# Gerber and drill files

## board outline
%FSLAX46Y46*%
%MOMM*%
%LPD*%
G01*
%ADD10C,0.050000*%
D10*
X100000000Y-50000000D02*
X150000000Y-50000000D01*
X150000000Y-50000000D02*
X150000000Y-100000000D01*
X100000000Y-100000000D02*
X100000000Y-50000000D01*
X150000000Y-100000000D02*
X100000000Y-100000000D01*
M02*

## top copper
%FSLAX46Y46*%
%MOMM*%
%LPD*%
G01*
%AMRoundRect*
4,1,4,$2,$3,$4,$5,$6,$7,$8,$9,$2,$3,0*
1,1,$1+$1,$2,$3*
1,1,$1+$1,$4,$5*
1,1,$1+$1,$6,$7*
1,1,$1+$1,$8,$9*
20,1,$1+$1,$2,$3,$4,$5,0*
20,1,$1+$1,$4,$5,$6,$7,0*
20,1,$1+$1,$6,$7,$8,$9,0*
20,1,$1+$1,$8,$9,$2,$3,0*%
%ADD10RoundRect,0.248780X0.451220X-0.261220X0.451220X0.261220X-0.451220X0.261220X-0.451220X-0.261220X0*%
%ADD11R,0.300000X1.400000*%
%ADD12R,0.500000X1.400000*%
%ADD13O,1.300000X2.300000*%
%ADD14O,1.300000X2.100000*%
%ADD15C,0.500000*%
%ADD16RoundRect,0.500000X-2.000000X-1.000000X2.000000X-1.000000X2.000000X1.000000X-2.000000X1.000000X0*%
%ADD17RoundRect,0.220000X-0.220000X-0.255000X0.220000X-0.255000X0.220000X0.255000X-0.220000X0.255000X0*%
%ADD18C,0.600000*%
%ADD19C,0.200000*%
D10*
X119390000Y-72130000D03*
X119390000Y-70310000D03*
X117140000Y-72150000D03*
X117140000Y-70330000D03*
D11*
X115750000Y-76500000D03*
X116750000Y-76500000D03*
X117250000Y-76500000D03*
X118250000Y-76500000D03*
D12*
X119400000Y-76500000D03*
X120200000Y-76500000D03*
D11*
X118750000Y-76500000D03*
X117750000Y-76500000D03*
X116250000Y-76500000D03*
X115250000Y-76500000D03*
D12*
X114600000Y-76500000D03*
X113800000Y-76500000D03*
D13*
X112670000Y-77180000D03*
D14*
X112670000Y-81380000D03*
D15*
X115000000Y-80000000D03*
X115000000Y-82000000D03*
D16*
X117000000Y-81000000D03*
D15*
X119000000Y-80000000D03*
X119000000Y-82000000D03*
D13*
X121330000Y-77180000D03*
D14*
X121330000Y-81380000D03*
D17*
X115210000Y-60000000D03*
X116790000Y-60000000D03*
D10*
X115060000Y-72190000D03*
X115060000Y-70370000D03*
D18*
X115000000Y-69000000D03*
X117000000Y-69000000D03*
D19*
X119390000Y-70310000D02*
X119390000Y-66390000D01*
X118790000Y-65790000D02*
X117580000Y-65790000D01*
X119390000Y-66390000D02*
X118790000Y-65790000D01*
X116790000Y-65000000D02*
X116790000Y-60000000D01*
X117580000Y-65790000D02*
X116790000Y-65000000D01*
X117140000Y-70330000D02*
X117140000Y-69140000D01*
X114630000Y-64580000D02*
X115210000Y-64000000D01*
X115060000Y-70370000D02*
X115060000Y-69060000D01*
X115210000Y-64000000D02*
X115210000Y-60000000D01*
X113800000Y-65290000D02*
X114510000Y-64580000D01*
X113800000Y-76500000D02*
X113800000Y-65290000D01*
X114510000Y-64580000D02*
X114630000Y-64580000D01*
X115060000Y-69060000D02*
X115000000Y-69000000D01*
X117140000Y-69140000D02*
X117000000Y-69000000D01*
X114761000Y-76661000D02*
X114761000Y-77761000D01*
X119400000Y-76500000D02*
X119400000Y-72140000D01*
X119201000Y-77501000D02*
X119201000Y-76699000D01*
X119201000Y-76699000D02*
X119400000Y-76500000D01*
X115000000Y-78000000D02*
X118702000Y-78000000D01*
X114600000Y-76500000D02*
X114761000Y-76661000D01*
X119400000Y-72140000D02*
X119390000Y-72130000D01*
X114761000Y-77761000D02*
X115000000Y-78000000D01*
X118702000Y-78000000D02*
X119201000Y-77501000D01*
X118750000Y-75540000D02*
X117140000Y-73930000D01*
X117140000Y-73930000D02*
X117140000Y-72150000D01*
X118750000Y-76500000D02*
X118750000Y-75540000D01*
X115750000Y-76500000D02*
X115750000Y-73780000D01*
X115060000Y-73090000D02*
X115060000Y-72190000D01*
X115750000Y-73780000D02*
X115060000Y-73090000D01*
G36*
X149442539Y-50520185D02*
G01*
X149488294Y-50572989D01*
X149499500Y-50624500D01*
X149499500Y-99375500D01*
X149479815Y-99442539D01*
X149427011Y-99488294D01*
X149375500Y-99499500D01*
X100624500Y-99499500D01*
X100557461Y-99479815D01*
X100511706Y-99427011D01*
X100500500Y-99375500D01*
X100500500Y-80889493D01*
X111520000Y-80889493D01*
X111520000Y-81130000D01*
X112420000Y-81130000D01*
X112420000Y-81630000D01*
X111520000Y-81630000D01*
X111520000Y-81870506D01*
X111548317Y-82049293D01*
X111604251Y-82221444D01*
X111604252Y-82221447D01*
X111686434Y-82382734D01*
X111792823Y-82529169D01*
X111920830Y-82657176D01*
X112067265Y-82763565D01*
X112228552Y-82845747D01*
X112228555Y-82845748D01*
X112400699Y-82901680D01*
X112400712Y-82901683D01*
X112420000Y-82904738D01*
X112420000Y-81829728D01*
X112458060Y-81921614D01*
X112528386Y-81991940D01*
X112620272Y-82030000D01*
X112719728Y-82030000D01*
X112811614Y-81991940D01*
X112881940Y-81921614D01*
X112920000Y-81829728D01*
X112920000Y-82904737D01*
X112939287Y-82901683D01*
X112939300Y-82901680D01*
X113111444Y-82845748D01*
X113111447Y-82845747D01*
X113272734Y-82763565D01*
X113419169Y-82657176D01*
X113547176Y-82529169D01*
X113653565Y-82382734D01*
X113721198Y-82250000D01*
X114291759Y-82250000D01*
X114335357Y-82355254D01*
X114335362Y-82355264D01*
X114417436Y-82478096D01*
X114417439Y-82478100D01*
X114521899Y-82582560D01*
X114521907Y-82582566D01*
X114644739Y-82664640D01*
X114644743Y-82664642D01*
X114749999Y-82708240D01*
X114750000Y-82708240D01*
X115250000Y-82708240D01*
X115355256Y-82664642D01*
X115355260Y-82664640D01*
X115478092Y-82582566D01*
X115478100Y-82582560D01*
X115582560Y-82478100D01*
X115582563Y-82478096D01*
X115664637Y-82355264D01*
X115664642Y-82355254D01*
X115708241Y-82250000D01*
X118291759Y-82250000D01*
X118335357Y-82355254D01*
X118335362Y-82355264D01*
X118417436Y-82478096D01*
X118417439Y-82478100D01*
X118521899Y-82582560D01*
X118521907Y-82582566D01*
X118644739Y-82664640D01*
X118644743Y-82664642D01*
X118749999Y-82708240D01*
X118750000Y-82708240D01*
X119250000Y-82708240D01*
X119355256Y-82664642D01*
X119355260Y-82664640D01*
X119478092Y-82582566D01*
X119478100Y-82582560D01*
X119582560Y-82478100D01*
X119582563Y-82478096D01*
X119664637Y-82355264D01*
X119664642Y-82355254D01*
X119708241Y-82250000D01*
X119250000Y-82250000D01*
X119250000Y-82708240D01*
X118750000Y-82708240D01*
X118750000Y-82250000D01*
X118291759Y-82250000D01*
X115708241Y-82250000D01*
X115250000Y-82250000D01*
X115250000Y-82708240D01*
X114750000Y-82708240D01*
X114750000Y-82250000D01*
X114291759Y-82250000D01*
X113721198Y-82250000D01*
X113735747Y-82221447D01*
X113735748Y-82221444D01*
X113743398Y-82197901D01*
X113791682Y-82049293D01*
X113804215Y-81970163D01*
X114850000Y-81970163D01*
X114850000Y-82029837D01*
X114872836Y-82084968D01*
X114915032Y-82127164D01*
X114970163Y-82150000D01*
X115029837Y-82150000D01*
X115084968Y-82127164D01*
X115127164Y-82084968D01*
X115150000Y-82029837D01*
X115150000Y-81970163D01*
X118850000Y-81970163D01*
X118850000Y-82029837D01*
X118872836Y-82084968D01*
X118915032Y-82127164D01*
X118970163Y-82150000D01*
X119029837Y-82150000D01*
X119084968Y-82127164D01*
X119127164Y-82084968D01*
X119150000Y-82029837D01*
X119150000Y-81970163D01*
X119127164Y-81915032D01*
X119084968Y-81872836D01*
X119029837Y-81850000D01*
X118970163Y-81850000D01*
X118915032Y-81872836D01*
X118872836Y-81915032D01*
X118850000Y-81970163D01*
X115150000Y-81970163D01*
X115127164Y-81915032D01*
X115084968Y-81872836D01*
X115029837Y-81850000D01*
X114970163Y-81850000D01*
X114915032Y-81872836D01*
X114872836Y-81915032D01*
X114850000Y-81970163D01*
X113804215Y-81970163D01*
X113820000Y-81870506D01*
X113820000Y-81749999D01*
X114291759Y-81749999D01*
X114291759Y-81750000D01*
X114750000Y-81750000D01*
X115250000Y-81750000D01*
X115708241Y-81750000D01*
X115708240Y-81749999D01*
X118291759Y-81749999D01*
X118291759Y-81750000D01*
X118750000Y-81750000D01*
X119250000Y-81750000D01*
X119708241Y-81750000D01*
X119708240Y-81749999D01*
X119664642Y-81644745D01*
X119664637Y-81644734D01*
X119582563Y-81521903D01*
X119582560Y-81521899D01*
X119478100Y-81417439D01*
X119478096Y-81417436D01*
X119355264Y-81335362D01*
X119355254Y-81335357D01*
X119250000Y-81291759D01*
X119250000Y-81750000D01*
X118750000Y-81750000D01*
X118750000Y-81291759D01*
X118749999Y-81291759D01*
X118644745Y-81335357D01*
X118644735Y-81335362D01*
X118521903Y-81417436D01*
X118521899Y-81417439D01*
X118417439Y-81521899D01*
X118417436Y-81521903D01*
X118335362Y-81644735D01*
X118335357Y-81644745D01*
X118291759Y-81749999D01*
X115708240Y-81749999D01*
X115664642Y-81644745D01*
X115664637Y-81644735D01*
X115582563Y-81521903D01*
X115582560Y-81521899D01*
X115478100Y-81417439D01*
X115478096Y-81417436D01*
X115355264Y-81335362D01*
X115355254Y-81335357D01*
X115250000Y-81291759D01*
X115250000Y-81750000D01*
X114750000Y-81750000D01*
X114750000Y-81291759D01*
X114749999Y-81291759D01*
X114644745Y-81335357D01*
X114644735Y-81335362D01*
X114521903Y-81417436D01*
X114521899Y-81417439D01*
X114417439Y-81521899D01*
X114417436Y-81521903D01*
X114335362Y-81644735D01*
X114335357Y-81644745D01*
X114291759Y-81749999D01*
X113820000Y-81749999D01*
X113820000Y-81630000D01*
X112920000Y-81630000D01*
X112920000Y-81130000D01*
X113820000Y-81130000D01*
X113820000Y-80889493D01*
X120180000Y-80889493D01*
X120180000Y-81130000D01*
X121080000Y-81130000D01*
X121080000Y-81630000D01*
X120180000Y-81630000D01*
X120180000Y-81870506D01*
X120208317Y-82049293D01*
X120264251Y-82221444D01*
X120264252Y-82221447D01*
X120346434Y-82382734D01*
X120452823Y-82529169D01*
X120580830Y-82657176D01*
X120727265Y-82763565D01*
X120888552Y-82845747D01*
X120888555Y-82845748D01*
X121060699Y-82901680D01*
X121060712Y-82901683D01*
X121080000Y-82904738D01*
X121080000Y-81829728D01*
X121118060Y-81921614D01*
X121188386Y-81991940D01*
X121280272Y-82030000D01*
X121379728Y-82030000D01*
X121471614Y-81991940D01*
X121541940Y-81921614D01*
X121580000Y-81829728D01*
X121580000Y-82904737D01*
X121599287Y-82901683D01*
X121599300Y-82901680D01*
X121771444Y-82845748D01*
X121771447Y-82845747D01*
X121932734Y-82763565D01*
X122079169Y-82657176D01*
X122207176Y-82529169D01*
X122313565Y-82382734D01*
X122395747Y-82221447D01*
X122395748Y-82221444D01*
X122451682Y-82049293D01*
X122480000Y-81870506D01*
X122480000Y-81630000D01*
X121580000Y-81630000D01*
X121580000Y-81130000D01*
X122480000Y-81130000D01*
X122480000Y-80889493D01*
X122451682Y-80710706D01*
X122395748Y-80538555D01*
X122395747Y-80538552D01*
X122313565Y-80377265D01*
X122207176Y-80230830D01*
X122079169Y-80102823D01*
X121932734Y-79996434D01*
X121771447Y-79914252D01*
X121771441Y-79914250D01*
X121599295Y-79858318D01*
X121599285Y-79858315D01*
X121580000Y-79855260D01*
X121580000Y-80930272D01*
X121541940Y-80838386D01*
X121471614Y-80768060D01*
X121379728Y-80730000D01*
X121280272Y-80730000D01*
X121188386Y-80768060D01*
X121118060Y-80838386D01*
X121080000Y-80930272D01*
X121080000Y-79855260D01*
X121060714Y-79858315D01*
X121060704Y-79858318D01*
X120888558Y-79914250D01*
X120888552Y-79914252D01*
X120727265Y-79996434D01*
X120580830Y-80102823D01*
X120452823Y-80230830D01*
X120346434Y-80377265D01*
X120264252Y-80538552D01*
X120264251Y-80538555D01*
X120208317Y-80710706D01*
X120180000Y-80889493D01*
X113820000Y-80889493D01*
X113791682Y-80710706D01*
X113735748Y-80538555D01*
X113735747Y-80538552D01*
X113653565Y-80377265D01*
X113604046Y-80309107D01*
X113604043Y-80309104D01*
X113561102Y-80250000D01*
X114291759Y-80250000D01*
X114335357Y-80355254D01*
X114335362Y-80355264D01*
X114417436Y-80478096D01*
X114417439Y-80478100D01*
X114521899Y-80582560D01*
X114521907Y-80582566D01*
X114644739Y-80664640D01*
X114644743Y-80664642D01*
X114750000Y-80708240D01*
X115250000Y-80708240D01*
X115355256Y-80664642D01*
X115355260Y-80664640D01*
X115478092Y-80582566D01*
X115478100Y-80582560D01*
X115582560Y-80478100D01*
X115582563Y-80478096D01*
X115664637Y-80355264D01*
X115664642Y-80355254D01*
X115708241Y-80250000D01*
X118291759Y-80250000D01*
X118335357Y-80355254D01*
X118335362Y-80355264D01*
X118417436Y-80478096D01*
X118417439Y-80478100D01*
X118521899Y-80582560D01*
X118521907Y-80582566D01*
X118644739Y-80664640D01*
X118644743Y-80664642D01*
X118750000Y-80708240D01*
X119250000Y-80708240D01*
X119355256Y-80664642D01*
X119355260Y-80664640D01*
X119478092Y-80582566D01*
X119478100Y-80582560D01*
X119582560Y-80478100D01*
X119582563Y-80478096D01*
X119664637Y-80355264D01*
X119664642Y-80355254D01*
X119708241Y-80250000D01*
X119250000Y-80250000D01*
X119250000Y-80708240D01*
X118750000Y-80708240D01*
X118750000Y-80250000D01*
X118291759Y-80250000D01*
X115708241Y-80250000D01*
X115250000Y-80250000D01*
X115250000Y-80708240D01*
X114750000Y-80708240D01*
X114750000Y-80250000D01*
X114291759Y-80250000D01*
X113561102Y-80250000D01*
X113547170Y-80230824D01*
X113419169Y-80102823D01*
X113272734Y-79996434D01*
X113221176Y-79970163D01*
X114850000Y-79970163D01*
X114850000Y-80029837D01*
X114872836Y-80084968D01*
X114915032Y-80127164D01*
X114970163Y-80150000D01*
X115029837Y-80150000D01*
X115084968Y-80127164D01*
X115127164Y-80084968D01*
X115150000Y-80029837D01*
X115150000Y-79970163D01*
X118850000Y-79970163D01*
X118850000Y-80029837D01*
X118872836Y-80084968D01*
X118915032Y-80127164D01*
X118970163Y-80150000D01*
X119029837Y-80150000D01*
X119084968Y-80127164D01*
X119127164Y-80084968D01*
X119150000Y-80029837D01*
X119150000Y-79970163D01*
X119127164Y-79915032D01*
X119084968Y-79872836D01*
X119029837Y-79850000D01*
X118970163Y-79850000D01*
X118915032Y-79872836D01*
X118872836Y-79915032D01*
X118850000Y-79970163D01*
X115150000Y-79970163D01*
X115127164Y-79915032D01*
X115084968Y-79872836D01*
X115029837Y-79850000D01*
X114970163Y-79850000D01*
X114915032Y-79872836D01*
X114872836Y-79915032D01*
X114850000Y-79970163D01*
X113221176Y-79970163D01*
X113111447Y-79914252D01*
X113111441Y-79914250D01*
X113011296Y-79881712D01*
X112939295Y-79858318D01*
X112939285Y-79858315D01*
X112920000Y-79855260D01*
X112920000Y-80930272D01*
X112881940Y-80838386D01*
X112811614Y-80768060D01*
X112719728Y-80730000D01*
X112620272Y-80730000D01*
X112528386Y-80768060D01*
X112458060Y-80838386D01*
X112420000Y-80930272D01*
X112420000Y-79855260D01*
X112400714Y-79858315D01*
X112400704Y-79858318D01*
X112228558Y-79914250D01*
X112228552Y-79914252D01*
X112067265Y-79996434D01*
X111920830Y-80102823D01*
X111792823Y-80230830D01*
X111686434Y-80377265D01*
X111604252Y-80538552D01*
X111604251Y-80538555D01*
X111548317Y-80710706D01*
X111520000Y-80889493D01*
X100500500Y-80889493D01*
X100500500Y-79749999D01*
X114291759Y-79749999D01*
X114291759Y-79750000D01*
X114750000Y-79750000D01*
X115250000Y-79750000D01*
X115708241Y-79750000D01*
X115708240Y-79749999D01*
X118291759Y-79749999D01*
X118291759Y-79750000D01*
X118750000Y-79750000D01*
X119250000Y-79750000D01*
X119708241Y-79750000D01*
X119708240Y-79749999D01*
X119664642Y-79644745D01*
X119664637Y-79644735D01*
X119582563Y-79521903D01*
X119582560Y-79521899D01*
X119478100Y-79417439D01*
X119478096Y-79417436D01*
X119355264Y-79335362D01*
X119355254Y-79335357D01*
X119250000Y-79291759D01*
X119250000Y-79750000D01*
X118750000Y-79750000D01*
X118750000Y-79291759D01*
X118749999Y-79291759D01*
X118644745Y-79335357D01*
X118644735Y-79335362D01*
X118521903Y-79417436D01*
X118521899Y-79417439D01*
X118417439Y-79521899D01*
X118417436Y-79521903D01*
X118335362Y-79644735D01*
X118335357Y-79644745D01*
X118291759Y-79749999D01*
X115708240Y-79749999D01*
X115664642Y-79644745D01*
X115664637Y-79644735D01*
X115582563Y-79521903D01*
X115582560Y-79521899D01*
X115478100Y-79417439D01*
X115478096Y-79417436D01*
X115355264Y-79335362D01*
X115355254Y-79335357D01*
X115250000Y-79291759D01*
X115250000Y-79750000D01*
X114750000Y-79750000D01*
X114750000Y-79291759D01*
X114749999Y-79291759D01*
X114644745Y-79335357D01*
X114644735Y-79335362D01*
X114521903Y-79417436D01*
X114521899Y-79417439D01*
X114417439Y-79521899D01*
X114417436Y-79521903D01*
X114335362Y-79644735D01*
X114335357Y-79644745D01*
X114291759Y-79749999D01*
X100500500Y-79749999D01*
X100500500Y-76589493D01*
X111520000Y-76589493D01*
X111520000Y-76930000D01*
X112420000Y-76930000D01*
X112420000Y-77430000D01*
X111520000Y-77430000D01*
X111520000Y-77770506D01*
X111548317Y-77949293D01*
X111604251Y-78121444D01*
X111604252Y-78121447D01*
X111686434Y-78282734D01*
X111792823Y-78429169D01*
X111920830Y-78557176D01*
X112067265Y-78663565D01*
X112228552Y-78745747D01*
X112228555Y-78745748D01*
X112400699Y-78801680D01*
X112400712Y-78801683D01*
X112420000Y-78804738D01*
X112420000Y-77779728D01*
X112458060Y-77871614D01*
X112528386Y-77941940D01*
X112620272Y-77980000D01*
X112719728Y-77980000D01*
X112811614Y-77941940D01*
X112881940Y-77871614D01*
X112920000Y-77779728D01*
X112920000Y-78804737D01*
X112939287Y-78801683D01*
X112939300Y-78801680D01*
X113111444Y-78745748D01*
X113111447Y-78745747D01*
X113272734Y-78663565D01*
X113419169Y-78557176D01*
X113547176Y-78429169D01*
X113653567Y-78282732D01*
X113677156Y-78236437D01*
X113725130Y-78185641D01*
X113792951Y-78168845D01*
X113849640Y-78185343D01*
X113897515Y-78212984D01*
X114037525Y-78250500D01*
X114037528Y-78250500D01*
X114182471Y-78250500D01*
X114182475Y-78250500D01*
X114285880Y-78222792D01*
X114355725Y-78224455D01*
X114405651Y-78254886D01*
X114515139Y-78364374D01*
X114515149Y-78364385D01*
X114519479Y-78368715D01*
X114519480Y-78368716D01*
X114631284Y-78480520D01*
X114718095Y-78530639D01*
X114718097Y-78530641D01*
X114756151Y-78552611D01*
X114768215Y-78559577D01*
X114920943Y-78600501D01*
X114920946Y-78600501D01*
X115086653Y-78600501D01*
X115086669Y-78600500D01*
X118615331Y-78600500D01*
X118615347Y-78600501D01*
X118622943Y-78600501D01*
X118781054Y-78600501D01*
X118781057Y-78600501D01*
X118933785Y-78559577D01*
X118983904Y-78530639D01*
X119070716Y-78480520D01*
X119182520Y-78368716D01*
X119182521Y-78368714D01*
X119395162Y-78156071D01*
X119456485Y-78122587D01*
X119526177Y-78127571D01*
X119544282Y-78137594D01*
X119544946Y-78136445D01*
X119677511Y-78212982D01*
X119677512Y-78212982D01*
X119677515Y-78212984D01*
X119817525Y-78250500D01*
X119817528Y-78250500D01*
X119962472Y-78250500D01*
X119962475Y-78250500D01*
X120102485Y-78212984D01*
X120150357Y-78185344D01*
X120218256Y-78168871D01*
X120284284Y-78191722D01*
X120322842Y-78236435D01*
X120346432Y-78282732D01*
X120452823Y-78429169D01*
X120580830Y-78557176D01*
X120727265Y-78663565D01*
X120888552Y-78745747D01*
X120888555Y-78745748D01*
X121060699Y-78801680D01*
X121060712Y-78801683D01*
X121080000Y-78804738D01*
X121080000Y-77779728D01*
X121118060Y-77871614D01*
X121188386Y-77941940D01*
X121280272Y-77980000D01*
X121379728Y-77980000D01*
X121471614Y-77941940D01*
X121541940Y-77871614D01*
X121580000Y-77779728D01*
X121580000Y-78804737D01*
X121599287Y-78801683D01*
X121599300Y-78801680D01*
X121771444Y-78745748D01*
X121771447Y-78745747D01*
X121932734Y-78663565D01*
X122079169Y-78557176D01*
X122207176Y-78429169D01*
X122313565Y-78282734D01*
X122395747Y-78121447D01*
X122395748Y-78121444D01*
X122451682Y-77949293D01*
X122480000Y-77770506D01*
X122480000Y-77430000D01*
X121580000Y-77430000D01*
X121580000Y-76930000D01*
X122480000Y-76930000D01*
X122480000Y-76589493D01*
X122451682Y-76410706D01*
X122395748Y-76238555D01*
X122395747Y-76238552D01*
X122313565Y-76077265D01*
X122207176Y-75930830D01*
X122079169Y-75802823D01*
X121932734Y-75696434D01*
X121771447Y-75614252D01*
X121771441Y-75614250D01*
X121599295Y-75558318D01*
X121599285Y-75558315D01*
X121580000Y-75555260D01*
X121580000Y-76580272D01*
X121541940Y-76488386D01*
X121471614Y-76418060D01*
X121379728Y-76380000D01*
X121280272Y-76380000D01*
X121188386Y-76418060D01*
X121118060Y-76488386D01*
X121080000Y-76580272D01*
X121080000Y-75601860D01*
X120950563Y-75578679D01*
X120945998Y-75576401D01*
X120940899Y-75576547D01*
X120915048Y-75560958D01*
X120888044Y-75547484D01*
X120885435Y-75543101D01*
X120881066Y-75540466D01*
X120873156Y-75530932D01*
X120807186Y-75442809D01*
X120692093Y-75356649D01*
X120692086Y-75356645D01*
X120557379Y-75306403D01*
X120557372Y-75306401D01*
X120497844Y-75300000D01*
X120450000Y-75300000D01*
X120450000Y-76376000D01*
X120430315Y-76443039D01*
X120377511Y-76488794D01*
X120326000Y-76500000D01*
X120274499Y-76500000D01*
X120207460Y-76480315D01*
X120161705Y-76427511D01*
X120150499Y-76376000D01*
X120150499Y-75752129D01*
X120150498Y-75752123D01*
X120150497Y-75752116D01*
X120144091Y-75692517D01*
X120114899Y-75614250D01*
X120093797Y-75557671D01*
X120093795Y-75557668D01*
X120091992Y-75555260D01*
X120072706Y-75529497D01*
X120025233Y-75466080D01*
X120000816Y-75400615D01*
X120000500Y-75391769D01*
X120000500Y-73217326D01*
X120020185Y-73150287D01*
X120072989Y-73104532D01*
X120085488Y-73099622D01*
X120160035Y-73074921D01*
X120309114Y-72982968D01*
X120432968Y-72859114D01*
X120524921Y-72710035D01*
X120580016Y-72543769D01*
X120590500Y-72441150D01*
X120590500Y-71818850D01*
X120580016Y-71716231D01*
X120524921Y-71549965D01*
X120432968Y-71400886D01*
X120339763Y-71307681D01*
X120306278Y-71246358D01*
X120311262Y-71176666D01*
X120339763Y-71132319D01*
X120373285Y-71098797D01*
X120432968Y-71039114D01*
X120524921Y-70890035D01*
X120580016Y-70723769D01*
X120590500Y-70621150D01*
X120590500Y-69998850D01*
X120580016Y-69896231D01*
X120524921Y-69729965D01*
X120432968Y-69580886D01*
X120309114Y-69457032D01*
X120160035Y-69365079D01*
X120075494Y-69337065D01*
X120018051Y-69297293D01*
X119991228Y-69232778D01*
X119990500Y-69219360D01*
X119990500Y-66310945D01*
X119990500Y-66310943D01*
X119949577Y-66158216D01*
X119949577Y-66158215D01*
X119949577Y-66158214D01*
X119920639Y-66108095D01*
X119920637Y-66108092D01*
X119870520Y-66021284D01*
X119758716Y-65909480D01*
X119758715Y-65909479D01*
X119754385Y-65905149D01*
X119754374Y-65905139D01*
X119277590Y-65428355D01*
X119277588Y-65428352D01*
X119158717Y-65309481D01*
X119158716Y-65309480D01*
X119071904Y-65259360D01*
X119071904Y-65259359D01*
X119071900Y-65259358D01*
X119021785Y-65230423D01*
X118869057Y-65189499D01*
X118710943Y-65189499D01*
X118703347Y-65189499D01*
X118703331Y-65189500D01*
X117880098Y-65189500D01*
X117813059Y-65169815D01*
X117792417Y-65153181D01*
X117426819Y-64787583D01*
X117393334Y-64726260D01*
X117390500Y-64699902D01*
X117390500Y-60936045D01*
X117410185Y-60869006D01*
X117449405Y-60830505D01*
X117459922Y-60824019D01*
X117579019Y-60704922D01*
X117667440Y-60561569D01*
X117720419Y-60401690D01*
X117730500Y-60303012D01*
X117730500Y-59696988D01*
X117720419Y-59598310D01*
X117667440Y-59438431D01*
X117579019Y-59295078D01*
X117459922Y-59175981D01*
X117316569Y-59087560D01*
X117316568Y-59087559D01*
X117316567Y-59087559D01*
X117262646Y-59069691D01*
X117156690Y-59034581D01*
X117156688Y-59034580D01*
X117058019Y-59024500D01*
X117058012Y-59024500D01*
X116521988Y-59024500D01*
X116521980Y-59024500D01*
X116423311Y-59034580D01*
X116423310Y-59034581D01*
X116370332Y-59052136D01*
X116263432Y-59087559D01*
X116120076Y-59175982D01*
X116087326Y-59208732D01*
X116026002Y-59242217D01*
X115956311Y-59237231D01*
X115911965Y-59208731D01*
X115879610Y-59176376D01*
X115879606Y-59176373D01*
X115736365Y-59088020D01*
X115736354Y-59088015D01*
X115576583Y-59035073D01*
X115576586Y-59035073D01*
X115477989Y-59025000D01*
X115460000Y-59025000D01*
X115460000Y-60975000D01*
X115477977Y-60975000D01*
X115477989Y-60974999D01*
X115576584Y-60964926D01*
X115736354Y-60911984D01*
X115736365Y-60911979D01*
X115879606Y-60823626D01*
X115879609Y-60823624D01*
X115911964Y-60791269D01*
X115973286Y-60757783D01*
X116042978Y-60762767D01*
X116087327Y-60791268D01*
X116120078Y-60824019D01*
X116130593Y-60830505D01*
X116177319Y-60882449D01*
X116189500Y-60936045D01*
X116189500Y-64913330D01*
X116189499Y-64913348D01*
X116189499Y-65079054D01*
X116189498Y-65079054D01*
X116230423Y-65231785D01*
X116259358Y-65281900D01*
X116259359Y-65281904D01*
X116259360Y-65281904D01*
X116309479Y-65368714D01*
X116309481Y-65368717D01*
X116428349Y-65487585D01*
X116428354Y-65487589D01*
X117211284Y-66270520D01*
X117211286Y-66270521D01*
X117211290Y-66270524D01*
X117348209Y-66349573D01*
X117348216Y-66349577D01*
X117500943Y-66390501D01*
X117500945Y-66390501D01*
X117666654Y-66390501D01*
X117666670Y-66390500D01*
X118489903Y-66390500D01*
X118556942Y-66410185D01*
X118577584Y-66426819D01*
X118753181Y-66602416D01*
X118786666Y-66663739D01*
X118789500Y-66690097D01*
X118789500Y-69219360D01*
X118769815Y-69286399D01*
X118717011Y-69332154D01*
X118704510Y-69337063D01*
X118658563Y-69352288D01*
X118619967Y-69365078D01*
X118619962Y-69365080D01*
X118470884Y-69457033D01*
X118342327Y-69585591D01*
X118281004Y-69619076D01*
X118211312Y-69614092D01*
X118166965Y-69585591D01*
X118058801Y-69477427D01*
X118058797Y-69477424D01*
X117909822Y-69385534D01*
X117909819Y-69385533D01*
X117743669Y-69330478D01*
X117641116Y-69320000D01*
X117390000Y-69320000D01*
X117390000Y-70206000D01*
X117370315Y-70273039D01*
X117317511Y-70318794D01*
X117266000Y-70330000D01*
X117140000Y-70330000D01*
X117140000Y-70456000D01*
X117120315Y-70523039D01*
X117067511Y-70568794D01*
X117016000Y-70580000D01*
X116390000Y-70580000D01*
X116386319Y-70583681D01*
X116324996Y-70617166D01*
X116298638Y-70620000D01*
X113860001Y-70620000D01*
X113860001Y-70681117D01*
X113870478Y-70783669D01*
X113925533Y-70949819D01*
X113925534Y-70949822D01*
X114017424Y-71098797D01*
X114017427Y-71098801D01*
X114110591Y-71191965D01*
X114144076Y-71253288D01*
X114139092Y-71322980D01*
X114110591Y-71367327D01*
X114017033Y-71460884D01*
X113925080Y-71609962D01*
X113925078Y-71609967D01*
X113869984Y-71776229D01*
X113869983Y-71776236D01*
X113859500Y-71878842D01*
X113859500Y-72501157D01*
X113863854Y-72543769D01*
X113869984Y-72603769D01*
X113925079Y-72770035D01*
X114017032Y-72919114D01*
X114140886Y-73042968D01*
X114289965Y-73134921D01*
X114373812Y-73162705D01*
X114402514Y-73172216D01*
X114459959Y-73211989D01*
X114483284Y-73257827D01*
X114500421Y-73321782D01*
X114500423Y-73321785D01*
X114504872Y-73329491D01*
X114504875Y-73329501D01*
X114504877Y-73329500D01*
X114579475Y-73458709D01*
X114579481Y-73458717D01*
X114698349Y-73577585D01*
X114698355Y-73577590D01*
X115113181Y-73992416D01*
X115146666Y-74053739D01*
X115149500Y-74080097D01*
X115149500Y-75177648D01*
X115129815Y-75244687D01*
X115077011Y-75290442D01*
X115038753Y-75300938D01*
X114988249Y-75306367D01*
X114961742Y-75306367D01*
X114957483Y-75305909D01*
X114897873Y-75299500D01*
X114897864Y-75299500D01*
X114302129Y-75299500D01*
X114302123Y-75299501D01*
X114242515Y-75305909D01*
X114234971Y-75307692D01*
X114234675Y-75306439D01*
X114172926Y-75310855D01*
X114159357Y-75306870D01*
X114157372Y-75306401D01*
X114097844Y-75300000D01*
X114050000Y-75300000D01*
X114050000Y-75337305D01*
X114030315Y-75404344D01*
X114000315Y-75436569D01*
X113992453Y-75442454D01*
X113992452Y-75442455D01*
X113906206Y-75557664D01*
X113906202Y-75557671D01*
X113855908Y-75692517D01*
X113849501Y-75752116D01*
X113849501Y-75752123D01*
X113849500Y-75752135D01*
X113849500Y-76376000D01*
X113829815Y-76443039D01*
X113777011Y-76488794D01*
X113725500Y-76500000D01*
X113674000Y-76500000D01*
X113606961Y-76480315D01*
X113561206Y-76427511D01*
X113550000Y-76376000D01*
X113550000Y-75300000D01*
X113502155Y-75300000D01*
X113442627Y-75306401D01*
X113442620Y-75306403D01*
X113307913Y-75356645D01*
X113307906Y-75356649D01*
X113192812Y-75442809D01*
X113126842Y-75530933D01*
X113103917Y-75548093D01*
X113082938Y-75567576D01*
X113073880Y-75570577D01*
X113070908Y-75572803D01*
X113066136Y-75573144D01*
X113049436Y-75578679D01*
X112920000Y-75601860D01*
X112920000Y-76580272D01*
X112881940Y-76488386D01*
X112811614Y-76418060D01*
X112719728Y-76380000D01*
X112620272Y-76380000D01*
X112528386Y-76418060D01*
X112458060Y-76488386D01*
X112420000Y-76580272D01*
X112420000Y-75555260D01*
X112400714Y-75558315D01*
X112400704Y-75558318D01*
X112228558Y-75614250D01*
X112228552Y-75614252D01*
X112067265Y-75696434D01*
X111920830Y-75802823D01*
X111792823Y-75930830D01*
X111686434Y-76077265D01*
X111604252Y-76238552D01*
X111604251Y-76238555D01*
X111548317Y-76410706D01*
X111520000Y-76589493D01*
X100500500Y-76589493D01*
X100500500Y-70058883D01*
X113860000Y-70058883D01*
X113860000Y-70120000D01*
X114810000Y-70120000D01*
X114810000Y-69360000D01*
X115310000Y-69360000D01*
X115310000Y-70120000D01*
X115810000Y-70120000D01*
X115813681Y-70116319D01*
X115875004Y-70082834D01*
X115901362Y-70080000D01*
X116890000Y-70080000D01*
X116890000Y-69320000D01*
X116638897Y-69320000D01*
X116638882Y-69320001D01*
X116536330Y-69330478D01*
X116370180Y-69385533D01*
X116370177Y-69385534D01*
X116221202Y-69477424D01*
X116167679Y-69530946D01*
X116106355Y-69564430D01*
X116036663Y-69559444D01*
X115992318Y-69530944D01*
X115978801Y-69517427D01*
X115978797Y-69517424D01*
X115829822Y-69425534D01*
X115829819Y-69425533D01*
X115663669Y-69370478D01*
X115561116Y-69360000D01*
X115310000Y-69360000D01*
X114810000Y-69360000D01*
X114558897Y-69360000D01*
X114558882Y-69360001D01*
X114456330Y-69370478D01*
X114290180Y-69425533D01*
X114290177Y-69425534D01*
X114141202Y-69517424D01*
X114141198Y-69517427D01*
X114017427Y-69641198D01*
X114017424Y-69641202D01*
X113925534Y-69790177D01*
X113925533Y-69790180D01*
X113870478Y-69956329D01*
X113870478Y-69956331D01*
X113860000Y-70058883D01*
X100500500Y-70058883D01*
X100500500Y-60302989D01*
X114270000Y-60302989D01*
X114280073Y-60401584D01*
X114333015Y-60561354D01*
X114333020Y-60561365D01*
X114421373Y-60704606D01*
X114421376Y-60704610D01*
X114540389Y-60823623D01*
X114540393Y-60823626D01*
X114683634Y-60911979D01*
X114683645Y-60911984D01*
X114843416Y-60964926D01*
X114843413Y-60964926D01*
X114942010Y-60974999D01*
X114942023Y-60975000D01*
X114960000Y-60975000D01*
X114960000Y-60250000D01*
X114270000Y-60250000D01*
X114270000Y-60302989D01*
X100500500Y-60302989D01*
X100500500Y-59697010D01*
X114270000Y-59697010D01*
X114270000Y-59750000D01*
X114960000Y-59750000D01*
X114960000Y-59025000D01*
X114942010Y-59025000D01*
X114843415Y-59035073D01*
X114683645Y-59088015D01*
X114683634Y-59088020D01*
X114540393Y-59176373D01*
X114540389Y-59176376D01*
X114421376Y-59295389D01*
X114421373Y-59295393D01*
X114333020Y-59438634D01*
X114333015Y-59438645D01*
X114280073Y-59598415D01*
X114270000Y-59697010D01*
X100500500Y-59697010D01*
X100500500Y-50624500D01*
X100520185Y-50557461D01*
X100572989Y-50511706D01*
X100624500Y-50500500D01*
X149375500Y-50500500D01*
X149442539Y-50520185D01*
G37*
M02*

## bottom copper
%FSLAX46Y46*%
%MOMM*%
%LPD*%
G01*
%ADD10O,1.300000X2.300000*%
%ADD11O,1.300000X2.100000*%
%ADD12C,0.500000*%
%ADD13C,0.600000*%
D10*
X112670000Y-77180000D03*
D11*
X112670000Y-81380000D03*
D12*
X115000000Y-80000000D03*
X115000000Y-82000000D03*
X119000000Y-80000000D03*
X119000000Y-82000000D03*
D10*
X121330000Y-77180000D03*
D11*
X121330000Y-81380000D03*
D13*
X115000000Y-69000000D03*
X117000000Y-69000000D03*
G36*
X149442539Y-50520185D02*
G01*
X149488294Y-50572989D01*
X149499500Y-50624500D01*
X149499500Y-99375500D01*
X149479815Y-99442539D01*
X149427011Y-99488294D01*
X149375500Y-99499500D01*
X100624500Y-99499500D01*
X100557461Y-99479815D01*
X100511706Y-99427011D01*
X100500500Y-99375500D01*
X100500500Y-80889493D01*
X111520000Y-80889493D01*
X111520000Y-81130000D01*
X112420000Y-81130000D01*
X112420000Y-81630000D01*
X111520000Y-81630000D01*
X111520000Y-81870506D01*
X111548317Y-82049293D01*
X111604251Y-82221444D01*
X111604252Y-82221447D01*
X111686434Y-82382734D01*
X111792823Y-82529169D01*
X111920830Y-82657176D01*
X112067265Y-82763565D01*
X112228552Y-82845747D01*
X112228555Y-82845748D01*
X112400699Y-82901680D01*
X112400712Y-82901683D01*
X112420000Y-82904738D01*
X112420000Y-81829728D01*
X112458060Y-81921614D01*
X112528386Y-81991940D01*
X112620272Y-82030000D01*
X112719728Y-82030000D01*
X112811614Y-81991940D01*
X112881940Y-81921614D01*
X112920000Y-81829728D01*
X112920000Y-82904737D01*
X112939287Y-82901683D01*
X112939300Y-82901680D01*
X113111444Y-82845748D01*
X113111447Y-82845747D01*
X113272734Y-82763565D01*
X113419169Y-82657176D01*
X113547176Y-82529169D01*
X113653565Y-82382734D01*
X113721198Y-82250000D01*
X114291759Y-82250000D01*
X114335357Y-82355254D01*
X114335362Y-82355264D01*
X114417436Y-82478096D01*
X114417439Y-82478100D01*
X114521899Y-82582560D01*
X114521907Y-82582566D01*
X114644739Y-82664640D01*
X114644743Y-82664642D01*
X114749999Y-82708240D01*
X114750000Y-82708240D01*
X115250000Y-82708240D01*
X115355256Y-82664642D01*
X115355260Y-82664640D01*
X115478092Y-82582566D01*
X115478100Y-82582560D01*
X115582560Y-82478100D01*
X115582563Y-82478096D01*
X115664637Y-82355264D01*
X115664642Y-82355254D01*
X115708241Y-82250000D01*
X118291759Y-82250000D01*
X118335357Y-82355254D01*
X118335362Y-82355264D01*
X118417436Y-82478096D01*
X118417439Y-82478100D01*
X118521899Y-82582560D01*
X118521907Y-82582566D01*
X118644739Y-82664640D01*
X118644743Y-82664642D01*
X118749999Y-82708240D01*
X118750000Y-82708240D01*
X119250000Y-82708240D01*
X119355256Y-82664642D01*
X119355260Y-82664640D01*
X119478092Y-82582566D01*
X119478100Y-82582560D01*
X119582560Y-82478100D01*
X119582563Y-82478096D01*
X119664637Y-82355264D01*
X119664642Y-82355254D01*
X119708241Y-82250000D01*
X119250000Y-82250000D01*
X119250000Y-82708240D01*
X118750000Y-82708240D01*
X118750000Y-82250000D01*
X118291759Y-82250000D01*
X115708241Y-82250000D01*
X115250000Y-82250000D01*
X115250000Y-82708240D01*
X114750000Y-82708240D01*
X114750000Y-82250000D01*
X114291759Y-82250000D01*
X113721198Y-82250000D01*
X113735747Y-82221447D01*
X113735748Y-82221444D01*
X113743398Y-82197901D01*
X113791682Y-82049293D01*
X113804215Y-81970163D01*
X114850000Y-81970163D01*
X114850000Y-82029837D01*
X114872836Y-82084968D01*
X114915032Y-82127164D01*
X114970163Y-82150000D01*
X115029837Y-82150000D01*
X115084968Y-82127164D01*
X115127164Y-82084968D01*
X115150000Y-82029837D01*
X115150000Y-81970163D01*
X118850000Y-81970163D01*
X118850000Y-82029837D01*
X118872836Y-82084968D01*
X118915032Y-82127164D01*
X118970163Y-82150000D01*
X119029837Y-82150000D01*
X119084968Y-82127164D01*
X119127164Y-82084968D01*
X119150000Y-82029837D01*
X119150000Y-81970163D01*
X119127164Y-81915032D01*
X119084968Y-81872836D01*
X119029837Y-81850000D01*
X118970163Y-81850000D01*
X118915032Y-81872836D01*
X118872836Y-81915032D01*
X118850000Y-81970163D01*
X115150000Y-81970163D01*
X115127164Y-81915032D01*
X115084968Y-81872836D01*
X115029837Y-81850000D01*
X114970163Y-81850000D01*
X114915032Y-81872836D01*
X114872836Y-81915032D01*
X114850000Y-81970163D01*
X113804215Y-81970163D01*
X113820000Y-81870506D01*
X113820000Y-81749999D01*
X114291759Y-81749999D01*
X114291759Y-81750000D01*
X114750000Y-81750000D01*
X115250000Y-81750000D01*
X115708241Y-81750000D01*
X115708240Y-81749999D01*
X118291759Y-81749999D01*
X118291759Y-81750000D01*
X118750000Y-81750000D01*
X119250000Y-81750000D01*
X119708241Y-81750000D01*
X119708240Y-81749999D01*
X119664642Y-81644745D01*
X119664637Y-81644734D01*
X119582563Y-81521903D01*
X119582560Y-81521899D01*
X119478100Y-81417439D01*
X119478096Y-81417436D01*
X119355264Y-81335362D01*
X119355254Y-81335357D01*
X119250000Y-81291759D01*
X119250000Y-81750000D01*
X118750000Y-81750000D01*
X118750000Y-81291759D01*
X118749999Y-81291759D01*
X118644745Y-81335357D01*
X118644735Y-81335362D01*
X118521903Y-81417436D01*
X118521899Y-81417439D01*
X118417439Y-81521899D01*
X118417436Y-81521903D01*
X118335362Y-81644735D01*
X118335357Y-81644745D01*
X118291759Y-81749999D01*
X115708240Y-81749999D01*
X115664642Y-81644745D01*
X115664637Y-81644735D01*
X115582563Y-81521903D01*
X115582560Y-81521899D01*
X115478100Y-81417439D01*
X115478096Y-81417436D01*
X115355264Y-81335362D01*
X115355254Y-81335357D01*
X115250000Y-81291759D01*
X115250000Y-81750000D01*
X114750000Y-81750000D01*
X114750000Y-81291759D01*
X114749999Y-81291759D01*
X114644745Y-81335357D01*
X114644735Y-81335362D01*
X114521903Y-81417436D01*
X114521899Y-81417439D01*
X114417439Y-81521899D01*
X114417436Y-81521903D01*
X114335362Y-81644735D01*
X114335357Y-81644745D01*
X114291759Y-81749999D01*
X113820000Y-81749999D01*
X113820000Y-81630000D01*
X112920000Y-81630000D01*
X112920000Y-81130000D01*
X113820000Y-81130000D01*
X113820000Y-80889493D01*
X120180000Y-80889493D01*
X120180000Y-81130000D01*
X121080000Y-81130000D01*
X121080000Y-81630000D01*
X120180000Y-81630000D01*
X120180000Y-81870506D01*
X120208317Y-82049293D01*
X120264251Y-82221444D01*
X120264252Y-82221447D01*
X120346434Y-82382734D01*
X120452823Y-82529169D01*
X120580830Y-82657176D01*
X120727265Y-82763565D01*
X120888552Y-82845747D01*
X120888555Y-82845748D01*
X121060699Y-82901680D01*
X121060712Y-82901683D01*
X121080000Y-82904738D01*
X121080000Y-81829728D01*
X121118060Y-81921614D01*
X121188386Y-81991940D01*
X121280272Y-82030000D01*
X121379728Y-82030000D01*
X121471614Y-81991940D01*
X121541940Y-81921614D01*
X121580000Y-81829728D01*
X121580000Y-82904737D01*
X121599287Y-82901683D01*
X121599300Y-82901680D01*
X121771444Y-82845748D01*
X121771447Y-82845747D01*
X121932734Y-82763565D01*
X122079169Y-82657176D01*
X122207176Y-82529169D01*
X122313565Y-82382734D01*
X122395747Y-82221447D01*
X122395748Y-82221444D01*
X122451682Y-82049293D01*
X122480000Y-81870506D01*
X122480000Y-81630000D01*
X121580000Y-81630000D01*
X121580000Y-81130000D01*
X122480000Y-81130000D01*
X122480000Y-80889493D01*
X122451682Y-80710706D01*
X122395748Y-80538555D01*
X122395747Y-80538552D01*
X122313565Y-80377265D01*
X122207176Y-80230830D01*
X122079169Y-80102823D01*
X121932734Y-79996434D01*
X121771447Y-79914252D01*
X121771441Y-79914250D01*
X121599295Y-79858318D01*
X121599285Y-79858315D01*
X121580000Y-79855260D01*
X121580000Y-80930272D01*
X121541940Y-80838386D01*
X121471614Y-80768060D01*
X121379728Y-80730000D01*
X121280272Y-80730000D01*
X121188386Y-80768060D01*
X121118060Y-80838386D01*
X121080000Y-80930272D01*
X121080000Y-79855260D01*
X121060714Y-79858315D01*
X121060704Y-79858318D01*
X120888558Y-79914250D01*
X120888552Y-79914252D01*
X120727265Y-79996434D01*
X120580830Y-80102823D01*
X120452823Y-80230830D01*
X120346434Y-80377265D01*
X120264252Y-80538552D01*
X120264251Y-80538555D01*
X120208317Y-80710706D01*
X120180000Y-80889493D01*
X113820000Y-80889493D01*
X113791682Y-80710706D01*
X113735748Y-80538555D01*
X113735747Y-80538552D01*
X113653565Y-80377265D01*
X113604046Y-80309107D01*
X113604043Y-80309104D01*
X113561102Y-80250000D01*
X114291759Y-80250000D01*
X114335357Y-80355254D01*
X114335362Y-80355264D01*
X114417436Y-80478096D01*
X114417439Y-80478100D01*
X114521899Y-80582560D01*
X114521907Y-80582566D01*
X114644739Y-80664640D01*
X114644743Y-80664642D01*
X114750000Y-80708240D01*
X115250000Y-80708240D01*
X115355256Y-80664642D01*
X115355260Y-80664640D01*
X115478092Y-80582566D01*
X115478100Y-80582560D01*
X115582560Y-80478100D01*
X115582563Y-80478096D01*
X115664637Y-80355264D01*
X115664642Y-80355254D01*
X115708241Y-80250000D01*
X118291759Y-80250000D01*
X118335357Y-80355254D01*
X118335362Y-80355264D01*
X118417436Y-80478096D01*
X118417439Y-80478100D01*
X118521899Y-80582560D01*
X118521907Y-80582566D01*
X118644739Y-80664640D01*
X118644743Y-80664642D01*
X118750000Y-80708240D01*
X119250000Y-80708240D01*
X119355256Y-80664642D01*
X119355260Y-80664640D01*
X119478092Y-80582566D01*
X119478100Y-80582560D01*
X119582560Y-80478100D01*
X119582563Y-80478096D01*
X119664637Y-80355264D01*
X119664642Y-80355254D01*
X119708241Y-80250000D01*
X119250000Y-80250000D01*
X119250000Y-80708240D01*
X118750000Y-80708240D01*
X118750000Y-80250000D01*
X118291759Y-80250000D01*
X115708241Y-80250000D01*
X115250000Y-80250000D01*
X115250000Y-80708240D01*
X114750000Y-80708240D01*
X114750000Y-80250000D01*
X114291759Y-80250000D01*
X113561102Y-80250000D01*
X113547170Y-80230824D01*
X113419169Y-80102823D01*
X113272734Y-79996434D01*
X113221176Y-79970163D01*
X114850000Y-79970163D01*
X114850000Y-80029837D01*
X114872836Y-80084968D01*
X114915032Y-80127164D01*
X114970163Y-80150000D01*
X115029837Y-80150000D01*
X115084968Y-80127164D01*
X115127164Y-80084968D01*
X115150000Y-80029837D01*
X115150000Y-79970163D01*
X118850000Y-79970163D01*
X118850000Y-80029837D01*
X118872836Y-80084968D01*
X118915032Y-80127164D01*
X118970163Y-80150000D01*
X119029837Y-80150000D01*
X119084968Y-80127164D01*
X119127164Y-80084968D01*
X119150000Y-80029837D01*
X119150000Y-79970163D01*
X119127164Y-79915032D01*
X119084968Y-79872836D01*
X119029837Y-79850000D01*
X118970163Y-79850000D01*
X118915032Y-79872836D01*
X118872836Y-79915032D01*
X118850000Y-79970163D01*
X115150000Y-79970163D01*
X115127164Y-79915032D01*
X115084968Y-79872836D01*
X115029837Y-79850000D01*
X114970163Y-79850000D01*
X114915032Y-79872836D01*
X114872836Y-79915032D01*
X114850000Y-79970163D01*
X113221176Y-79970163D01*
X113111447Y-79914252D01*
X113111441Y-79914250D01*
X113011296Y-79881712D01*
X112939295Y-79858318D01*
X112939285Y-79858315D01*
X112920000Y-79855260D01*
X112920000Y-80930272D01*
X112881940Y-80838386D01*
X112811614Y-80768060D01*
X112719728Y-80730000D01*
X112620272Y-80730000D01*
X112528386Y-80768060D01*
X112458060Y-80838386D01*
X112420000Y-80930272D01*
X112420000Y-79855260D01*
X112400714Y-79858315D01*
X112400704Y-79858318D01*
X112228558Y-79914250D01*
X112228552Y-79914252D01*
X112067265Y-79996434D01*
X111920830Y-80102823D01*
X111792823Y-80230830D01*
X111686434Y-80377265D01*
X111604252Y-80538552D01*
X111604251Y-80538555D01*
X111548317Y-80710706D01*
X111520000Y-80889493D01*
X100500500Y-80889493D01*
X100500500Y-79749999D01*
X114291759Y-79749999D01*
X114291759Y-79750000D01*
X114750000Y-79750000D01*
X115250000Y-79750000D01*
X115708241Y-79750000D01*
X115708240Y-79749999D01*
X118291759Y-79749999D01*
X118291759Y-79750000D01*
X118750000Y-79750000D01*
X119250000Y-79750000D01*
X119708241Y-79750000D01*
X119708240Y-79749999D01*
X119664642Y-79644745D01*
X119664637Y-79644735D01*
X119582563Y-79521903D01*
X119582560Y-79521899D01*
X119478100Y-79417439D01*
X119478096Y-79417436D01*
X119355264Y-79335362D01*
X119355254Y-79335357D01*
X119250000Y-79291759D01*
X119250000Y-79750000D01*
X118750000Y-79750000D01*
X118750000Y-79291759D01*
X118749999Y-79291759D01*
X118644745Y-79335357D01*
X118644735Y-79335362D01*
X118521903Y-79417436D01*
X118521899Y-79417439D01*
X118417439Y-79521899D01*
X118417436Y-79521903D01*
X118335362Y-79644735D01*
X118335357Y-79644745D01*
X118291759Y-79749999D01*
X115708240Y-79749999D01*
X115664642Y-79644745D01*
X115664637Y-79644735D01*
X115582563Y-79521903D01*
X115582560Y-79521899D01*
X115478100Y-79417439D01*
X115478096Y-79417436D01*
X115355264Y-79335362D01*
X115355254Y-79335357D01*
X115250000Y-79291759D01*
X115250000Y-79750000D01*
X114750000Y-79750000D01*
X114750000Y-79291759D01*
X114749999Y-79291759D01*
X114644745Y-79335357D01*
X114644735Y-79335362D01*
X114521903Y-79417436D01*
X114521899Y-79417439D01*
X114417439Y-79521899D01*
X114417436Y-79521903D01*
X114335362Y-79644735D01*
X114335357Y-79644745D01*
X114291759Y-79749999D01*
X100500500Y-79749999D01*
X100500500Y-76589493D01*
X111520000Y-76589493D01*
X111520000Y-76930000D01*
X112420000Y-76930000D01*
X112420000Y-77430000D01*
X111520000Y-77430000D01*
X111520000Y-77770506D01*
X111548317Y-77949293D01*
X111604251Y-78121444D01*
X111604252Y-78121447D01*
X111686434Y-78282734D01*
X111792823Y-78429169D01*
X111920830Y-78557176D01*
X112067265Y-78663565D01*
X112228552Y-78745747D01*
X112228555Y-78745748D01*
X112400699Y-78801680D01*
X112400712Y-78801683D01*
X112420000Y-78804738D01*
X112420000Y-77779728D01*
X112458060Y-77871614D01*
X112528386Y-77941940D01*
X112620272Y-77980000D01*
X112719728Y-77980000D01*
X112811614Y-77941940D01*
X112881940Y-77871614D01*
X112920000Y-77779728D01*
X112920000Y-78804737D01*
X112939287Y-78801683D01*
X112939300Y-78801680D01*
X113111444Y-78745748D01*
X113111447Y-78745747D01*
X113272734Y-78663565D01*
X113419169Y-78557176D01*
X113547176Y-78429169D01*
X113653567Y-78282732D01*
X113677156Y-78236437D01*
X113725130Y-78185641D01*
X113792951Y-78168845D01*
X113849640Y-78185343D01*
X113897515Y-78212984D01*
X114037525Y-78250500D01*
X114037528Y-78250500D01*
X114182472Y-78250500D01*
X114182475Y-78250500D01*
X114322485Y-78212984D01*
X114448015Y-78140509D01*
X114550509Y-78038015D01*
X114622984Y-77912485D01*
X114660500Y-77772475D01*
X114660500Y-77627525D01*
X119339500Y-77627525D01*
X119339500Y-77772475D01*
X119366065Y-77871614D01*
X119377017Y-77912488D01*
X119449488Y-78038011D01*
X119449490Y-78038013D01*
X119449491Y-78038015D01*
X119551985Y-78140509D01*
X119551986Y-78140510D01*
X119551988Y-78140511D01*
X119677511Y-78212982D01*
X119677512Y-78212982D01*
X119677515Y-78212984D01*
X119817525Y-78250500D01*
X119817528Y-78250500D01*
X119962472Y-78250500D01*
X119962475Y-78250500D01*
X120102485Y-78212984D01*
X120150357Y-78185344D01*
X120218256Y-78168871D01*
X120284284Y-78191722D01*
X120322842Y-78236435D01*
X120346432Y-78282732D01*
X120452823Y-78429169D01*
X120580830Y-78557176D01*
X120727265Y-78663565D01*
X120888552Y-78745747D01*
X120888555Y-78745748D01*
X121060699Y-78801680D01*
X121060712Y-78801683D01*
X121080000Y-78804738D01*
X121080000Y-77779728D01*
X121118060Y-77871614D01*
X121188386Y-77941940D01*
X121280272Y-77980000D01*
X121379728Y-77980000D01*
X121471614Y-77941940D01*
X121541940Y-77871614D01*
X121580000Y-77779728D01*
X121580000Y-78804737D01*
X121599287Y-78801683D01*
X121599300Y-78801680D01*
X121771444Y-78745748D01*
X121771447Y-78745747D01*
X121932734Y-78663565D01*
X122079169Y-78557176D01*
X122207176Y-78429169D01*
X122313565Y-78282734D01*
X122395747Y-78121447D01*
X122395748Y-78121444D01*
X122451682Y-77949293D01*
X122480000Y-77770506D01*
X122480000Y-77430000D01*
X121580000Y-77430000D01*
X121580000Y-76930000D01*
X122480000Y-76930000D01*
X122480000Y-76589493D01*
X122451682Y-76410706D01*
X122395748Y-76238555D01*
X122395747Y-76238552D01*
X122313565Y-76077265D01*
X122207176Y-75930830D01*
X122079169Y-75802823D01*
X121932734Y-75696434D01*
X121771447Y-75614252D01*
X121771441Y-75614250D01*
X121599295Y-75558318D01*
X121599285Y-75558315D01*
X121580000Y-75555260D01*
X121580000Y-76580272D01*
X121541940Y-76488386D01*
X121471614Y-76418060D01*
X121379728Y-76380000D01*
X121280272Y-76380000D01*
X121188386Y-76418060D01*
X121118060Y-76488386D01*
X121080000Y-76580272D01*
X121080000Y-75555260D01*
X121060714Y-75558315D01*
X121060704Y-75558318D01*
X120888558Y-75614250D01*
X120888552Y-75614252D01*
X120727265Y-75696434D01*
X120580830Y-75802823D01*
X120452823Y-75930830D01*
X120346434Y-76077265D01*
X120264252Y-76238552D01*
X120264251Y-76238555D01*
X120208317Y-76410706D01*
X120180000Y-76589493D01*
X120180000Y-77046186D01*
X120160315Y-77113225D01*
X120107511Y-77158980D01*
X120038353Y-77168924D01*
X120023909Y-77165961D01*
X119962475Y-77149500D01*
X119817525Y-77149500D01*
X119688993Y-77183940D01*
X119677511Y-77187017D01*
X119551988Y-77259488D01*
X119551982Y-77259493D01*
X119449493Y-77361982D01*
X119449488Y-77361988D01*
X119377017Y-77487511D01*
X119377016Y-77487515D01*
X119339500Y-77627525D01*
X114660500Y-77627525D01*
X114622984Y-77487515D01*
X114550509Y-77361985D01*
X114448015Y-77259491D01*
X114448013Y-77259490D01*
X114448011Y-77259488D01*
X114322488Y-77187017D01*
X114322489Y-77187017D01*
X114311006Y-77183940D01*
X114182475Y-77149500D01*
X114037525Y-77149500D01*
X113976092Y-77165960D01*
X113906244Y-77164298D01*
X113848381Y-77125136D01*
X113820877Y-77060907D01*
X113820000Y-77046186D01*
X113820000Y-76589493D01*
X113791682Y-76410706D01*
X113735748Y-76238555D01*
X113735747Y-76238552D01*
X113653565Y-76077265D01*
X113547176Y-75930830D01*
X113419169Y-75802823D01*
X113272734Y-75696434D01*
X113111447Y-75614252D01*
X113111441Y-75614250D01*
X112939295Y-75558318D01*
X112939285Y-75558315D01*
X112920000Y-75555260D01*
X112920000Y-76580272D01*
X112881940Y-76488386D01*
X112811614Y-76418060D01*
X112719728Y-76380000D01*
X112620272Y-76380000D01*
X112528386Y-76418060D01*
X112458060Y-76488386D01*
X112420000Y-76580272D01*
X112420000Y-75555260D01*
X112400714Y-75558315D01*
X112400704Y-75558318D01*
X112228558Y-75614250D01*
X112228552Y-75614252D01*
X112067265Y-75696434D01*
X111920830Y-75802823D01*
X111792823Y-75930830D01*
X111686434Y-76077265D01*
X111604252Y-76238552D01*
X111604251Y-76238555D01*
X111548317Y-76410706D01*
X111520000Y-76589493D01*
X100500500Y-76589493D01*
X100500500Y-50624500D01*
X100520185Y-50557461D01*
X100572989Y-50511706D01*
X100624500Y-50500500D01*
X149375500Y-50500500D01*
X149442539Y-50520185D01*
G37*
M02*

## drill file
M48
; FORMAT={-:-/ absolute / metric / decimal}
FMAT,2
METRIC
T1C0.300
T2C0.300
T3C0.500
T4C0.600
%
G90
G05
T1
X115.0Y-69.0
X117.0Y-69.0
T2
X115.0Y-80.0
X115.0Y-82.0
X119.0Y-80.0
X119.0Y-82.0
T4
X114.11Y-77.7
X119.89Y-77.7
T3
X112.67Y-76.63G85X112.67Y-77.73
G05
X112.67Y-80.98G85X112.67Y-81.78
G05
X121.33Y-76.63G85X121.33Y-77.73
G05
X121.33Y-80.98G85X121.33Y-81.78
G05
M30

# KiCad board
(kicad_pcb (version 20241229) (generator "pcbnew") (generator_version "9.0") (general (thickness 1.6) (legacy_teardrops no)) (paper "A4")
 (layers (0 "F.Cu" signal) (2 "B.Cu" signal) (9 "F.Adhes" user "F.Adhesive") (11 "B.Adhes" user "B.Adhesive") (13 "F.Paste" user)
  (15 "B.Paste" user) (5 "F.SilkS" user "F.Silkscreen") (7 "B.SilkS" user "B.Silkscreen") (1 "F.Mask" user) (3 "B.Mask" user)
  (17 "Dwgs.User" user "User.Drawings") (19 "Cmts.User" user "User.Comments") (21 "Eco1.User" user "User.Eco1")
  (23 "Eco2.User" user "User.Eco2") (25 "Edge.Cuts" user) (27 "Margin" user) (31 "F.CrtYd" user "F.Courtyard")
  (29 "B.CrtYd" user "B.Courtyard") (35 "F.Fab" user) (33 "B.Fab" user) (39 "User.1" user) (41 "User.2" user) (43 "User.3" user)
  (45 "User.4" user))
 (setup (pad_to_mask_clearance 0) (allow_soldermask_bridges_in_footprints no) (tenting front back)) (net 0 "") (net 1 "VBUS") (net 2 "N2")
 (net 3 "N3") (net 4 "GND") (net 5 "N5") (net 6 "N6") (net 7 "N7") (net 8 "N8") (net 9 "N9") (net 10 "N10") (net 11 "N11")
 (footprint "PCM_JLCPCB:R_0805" (layer "F.Cu") (at 119.39 71.22 90)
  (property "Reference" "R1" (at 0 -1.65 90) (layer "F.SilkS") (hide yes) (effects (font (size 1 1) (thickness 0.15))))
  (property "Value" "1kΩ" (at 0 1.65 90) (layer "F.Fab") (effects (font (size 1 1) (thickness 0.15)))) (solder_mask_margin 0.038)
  (pad "1" smd roundrect (at -0.91 0 90) (size 1.02 1.4) (layers "F.Cu" "F.Mask" "F.Paste") (roundrect_rratio 0.243902) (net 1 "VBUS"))
  (pad "2" smd roundrect (at 0.91 0 90) (size 1.02 1.4) (layers "F.Cu" "F.Mask" "F.Paste") (roundrect_rratio 0.243902) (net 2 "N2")))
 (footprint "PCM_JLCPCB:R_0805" (layer "F.Cu") (at 117.14 71.24 90)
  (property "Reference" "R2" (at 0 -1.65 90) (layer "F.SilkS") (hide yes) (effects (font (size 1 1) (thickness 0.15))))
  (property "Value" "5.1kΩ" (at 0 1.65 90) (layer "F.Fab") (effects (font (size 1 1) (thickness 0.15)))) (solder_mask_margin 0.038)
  (pad "1" smd roundrect (at -0.91 0 90) (size 1.02 1.4) (layers "F.Cu" "F.Mask" "F.Paste") (roundrect_rratio 0.243902) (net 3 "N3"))
  (pad "2" smd roundrect (at 0.91 0 90) (size 1.02 1.4) (layers "F.Cu" "F.Mask" "F.Paste") (roundrect_rratio 0.243902) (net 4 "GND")))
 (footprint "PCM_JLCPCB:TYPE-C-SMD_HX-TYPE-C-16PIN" (layer "F.Cu") (at 117 79)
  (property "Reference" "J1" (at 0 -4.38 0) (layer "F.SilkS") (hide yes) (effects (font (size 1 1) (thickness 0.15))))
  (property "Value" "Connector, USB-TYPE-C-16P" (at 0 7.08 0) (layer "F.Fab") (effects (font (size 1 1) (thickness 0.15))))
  (pad "" np_thru_hole circle (at -2.89 -1.3) (size 0.6 0.6) (drill 0.6) (layers "*.Cu" "*.Mask"))
  (pad "" np_thru_hole circle (at 2.89 -1.3) (size 0.6 0.6) (drill 0.6) (layers "*.Cu" "*.Mask"))
  (pad "A5" smd rect (at -1.25 -2.5) (size 0.3 1.4) (layers "F.Cu" "F.Mask" "F.Paste") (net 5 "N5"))
  (pad "A6" smd rect (at -0.25 -2.5) (size 0.3 1.4) (layers "F.Cu" "F.Mask" "F.Paste") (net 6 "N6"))
  (pad "A7" smd rect (at 0.25 -2.5) (size 0.3 1.4) (layers "F.Cu" "F.Mask" "F.Paste") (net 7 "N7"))
  (pad "A8" smd rect (at 1.25 -2.5) (size 0.3 1.4) (layers "F.Cu" "F.Mask" "F.Paste") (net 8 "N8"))
  (pad "A9B4" smd rect (at 2.4 -2.5) (size 0.5 1.4) (layers "F.Cu" "F.Mask" "F.Paste") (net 1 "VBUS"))
  (pad "A12B1" smd rect (at 3.2 -2.5) (size 0.5 1.4) (layers "F.Cu" "F.Mask" "F.Paste") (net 4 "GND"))
  (pad "B5" smd rect (at 1.75 -2.5) (size 0.3 1.4) (layers "F.Cu" "F.Mask" "F.Paste") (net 3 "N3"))
  (pad "B6" smd rect (at 0.75 -2.5) (size 0.3 1.4) (layers "F.Cu" "F.Mask" "F.Paste") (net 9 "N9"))
  (pad "B7" smd rect (at -0.75 -2.5) (size 0.3 1.4) (layers "F.Cu" "F.Mask" "F.Paste") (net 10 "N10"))
  (pad "B8" smd rect (at -1.75 -2.5) (size 0.3 1.4) (layers "F.Cu" "F.Mask" "F.Paste") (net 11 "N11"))
  (pad "B9A4" smd rect (at -2.4 -2.5) (size 0.5 1.4) (layers "F.Cu" "F.Mask" "F.Paste") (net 1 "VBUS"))
  (pad "B12A1" smd rect (at -3.2 -2.5) (size 0.5 1.4) (layers "F.Cu" "F.Mask" "F.Paste") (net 4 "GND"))
  (pad "S1" thru_hole oval (at -4.33 -1.82) (size 1.3 2.3) (drill oval 0.5 1.6) (layers "*.Cu" "*.Mask") (remove_unused_layers no)
   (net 4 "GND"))
  (pad "S1" thru_hole oval (at -4.33 2.38) (size 1.3 2.1) (drill oval 0.5 1.3) (layers "*.Cu" "*.Mask") (remove_unused_layers no)
   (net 4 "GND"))
  (pad "S1" thru_hole circle (at -2 1) (size 0.5 0.5) (drill 0.3) (layers "*.Cu" "*.Mask") (remove_unused_layers no) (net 4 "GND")
   (thermal_bridge_angle 90))
  (pad "S1" thru_hole circle (at -2 3) (size 0.5 0.5) (drill 0.3) (layers "*.Cu" "*.Mask") (remove_unused_layers no) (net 4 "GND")
   (thermal_bridge_angle 90))
  (pad "S1" smd roundrect (at 0 2) (size 5 3) (layers "F.Cu" "F.Mask" "F.Paste") (roundrect_rratio 0.1666666667) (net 4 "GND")
   (zone_connect 2))
  (pad "S1" thru_hole circle (at 2 1) (size 0.5 0.5) (drill 0.3) (layers "*.Cu" "*.Mask") (remove_unused_layers no) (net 4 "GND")
   (thermal_bridge_angle 90))
  (pad "S1" thru_hole circle (at 2 3) (size 0.5 0.5) (drill 0.3) (layers "*.Cu" "*.Mask") (remove_unused_layers no) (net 4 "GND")
   (thermal_bridge_angle 90))
  (pad "S1" thru_hole oval (at 4.33 -1.82) (size 1.3 2.3) (drill oval 0.5 1.6) (layers "*.Cu" "*.Mask") (remove_unused_layers no)
   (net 4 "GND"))
  (pad "S1" thru_hole oval (at 4.33 2.38) (size 1.3 2.1) (drill oval 0.5 1.3) (layers "*.Cu" "*.Mask") (remove_unused_layers no)
   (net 4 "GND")))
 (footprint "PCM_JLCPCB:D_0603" (layer "F.Cu") (at 116 60)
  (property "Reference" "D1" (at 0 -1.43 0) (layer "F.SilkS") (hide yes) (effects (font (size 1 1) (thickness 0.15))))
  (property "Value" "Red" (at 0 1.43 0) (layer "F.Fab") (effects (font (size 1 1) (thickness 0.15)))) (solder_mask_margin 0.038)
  (pad "1" smd roundrect (at -0.79 0) (size 0.88 0.95) (layers "F.Cu" "F.Mask" "F.Paste") (roundrect_rratio 0.25) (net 4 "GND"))
  (pad "2" smd roundrect (at 0.79 0) (size 0.88 0.95) (layers "F.Cu" "F.Mask" "F.Paste") (roundrect_rratio 0.25) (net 2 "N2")))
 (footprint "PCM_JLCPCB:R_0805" (layer "F.Cu") (at 115.06 71.28 90)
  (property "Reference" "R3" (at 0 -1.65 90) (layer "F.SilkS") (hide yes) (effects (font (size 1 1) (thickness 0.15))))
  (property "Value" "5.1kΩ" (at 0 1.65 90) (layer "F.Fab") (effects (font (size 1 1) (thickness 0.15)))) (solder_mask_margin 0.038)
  (pad "1" smd roundrect (at -0.91 0 90) (size 1.02 1.4) (layers "F.Cu" "F.Mask" "F.Paste") (roundrect_rratio 0.243902) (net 5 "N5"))
  (pad "2" smd roundrect (at 0.91 0 90) (size 1.02 1.4) (layers "F.Cu" "F.Mask" "F.Paste") (roundrect_rratio 0.243902) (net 4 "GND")))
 (gr_line (start 100 50) (end 150 50) (stroke (width 0.05) (type default)) (layer "Edge.Cuts"))
 (gr_line (start 150 50) (end 150 100) (stroke (width 0.05) (type default)) (layer "Edge.Cuts"))
 (gr_line (start 100 100) (end 100 50) (stroke (width 0.05) (type default)) (layer "Edge.Cuts"))
 (gr_line (start 150 100) (end 100 100) (stroke (width 0.05) (type default)) (layer "Edge.Cuts"))
 (segment (start 119.39 70.31) (end 119.39 66.39) (width 0.2) (layer "F.Cu") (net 2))
 (segment (start 118.79 65.79) (end 117.58 65.79) (width 0.2) (layer "F.Cu") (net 2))
 (segment (start 119.39 66.39) (end 118.79 65.79) (width 0.2) (layer "F.Cu") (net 2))
 (segment (start 116.79 65) (end 116.79 60) (width 0.2) (layer "F.Cu") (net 2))
 (segment (start 117.58 65.79) (end 116.79 65) (width 0.2) (layer "F.Cu") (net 2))
 (segment (start 117.14 70.33) (end 117.14 69.14) (width 0.2) (layer "F.Cu") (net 4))
 (segment (start 114.63 64.58) (end 115.21 64) (width 0.2) (layer "F.Cu") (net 4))
 (segment (start 115.06 70.37) (end 115.06 69.06) (width 0.2) (layer "F.Cu") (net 4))
 (segment (start 115.21 64) (end 115.21 60) (width 0.2) (layer "F.Cu") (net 4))
 (segment (start 113.8 65.29) (end 114.51 64.58) (width 0.2) (layer "F.Cu") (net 4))
 (segment (start 113.8 76.5) (end 113.8 65.29) (width 0.2) (layer "F.Cu") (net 4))
 (segment (start 114.51 64.58) (end 114.63 64.58) (width 0.2) (layer "F.Cu") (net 4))
 (segment (start 115.06 69.06) (end 115 69) (width 0.2) (layer "F.Cu") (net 4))
 (segment (start 117.14 69.14) (end 117 69) (width 0.2) (layer "F.Cu") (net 4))
 (via (at 115 69) (size 0.6) (drill 0.3) (layers "F.Cu" "B.Cu") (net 4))
 (via (at 117 69) (size 0.6) (drill 0.3) (layers "F.Cu" "B.Cu") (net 4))
 (segment (start 114.761 76.661) (end 114.761 77.761) (width 0.2) (layer "F.Cu") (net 1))
 (segment (start 119.4 76.5) (end 119.4 72.14) (width 0.2) (layer "F.Cu") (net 1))
 (segment (start 119.201 77.501) (end 119.201 76.699) (width 0.2) (layer "F.Cu") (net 1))
 (segment (start 119.201 76.699) (end 119.4 76.5) (width 0.2) (layer "F.Cu") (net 1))
 (segment (start 115 78) (end 118.702 78) (width 0.2) (layer "F.Cu") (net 1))
 (segment (start 114.6 76.5) (end 114.761 76.661) (width 0.2) (layer "F.Cu") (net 1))
 (segment (start 119.4 72.14) (end 119.39 72.13) (width 0.2) (layer "F.Cu") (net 1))
 (segment (start 114.761 77.761) (end 115 78) (width 0.2) (layer "F.Cu") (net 1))
 (segment (start 118.702 78) (end 119.201 77.501) (width 0.2) (layer "F.Cu") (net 1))
 (segment (start 118.75 75.54) (end 117.14 73.93) (width 0.2) (layer "F.Cu") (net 3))
 (segment (start 117.14 73.93) (end 117.14 72.15) (width 0.2) (layer "F.Cu") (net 3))
 (segment (start 118.75 76.5) (end 118.75 75.54) (width 0.2) (layer "F.Cu") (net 3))
 (segment (start 115.75 76.5) (end 115.75 73.78) (width 0.2) (layer "F.Cu") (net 5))
 (segment (start 115.06 73.09) (end 115.06 72.19) (width 0.2) (layer "F.Cu") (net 5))
 (segment (start 115.75 73.78) (end 115.06 73.09) (width 0.2) (layer "F.Cu") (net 5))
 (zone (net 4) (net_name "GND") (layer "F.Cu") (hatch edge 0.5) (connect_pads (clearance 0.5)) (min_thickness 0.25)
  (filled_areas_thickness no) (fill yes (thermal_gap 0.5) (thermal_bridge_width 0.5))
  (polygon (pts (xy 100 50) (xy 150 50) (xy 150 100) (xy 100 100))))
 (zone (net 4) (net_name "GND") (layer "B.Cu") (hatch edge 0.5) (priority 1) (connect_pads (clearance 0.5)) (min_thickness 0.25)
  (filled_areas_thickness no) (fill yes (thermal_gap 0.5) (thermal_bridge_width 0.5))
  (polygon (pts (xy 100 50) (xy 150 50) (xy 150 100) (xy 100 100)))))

